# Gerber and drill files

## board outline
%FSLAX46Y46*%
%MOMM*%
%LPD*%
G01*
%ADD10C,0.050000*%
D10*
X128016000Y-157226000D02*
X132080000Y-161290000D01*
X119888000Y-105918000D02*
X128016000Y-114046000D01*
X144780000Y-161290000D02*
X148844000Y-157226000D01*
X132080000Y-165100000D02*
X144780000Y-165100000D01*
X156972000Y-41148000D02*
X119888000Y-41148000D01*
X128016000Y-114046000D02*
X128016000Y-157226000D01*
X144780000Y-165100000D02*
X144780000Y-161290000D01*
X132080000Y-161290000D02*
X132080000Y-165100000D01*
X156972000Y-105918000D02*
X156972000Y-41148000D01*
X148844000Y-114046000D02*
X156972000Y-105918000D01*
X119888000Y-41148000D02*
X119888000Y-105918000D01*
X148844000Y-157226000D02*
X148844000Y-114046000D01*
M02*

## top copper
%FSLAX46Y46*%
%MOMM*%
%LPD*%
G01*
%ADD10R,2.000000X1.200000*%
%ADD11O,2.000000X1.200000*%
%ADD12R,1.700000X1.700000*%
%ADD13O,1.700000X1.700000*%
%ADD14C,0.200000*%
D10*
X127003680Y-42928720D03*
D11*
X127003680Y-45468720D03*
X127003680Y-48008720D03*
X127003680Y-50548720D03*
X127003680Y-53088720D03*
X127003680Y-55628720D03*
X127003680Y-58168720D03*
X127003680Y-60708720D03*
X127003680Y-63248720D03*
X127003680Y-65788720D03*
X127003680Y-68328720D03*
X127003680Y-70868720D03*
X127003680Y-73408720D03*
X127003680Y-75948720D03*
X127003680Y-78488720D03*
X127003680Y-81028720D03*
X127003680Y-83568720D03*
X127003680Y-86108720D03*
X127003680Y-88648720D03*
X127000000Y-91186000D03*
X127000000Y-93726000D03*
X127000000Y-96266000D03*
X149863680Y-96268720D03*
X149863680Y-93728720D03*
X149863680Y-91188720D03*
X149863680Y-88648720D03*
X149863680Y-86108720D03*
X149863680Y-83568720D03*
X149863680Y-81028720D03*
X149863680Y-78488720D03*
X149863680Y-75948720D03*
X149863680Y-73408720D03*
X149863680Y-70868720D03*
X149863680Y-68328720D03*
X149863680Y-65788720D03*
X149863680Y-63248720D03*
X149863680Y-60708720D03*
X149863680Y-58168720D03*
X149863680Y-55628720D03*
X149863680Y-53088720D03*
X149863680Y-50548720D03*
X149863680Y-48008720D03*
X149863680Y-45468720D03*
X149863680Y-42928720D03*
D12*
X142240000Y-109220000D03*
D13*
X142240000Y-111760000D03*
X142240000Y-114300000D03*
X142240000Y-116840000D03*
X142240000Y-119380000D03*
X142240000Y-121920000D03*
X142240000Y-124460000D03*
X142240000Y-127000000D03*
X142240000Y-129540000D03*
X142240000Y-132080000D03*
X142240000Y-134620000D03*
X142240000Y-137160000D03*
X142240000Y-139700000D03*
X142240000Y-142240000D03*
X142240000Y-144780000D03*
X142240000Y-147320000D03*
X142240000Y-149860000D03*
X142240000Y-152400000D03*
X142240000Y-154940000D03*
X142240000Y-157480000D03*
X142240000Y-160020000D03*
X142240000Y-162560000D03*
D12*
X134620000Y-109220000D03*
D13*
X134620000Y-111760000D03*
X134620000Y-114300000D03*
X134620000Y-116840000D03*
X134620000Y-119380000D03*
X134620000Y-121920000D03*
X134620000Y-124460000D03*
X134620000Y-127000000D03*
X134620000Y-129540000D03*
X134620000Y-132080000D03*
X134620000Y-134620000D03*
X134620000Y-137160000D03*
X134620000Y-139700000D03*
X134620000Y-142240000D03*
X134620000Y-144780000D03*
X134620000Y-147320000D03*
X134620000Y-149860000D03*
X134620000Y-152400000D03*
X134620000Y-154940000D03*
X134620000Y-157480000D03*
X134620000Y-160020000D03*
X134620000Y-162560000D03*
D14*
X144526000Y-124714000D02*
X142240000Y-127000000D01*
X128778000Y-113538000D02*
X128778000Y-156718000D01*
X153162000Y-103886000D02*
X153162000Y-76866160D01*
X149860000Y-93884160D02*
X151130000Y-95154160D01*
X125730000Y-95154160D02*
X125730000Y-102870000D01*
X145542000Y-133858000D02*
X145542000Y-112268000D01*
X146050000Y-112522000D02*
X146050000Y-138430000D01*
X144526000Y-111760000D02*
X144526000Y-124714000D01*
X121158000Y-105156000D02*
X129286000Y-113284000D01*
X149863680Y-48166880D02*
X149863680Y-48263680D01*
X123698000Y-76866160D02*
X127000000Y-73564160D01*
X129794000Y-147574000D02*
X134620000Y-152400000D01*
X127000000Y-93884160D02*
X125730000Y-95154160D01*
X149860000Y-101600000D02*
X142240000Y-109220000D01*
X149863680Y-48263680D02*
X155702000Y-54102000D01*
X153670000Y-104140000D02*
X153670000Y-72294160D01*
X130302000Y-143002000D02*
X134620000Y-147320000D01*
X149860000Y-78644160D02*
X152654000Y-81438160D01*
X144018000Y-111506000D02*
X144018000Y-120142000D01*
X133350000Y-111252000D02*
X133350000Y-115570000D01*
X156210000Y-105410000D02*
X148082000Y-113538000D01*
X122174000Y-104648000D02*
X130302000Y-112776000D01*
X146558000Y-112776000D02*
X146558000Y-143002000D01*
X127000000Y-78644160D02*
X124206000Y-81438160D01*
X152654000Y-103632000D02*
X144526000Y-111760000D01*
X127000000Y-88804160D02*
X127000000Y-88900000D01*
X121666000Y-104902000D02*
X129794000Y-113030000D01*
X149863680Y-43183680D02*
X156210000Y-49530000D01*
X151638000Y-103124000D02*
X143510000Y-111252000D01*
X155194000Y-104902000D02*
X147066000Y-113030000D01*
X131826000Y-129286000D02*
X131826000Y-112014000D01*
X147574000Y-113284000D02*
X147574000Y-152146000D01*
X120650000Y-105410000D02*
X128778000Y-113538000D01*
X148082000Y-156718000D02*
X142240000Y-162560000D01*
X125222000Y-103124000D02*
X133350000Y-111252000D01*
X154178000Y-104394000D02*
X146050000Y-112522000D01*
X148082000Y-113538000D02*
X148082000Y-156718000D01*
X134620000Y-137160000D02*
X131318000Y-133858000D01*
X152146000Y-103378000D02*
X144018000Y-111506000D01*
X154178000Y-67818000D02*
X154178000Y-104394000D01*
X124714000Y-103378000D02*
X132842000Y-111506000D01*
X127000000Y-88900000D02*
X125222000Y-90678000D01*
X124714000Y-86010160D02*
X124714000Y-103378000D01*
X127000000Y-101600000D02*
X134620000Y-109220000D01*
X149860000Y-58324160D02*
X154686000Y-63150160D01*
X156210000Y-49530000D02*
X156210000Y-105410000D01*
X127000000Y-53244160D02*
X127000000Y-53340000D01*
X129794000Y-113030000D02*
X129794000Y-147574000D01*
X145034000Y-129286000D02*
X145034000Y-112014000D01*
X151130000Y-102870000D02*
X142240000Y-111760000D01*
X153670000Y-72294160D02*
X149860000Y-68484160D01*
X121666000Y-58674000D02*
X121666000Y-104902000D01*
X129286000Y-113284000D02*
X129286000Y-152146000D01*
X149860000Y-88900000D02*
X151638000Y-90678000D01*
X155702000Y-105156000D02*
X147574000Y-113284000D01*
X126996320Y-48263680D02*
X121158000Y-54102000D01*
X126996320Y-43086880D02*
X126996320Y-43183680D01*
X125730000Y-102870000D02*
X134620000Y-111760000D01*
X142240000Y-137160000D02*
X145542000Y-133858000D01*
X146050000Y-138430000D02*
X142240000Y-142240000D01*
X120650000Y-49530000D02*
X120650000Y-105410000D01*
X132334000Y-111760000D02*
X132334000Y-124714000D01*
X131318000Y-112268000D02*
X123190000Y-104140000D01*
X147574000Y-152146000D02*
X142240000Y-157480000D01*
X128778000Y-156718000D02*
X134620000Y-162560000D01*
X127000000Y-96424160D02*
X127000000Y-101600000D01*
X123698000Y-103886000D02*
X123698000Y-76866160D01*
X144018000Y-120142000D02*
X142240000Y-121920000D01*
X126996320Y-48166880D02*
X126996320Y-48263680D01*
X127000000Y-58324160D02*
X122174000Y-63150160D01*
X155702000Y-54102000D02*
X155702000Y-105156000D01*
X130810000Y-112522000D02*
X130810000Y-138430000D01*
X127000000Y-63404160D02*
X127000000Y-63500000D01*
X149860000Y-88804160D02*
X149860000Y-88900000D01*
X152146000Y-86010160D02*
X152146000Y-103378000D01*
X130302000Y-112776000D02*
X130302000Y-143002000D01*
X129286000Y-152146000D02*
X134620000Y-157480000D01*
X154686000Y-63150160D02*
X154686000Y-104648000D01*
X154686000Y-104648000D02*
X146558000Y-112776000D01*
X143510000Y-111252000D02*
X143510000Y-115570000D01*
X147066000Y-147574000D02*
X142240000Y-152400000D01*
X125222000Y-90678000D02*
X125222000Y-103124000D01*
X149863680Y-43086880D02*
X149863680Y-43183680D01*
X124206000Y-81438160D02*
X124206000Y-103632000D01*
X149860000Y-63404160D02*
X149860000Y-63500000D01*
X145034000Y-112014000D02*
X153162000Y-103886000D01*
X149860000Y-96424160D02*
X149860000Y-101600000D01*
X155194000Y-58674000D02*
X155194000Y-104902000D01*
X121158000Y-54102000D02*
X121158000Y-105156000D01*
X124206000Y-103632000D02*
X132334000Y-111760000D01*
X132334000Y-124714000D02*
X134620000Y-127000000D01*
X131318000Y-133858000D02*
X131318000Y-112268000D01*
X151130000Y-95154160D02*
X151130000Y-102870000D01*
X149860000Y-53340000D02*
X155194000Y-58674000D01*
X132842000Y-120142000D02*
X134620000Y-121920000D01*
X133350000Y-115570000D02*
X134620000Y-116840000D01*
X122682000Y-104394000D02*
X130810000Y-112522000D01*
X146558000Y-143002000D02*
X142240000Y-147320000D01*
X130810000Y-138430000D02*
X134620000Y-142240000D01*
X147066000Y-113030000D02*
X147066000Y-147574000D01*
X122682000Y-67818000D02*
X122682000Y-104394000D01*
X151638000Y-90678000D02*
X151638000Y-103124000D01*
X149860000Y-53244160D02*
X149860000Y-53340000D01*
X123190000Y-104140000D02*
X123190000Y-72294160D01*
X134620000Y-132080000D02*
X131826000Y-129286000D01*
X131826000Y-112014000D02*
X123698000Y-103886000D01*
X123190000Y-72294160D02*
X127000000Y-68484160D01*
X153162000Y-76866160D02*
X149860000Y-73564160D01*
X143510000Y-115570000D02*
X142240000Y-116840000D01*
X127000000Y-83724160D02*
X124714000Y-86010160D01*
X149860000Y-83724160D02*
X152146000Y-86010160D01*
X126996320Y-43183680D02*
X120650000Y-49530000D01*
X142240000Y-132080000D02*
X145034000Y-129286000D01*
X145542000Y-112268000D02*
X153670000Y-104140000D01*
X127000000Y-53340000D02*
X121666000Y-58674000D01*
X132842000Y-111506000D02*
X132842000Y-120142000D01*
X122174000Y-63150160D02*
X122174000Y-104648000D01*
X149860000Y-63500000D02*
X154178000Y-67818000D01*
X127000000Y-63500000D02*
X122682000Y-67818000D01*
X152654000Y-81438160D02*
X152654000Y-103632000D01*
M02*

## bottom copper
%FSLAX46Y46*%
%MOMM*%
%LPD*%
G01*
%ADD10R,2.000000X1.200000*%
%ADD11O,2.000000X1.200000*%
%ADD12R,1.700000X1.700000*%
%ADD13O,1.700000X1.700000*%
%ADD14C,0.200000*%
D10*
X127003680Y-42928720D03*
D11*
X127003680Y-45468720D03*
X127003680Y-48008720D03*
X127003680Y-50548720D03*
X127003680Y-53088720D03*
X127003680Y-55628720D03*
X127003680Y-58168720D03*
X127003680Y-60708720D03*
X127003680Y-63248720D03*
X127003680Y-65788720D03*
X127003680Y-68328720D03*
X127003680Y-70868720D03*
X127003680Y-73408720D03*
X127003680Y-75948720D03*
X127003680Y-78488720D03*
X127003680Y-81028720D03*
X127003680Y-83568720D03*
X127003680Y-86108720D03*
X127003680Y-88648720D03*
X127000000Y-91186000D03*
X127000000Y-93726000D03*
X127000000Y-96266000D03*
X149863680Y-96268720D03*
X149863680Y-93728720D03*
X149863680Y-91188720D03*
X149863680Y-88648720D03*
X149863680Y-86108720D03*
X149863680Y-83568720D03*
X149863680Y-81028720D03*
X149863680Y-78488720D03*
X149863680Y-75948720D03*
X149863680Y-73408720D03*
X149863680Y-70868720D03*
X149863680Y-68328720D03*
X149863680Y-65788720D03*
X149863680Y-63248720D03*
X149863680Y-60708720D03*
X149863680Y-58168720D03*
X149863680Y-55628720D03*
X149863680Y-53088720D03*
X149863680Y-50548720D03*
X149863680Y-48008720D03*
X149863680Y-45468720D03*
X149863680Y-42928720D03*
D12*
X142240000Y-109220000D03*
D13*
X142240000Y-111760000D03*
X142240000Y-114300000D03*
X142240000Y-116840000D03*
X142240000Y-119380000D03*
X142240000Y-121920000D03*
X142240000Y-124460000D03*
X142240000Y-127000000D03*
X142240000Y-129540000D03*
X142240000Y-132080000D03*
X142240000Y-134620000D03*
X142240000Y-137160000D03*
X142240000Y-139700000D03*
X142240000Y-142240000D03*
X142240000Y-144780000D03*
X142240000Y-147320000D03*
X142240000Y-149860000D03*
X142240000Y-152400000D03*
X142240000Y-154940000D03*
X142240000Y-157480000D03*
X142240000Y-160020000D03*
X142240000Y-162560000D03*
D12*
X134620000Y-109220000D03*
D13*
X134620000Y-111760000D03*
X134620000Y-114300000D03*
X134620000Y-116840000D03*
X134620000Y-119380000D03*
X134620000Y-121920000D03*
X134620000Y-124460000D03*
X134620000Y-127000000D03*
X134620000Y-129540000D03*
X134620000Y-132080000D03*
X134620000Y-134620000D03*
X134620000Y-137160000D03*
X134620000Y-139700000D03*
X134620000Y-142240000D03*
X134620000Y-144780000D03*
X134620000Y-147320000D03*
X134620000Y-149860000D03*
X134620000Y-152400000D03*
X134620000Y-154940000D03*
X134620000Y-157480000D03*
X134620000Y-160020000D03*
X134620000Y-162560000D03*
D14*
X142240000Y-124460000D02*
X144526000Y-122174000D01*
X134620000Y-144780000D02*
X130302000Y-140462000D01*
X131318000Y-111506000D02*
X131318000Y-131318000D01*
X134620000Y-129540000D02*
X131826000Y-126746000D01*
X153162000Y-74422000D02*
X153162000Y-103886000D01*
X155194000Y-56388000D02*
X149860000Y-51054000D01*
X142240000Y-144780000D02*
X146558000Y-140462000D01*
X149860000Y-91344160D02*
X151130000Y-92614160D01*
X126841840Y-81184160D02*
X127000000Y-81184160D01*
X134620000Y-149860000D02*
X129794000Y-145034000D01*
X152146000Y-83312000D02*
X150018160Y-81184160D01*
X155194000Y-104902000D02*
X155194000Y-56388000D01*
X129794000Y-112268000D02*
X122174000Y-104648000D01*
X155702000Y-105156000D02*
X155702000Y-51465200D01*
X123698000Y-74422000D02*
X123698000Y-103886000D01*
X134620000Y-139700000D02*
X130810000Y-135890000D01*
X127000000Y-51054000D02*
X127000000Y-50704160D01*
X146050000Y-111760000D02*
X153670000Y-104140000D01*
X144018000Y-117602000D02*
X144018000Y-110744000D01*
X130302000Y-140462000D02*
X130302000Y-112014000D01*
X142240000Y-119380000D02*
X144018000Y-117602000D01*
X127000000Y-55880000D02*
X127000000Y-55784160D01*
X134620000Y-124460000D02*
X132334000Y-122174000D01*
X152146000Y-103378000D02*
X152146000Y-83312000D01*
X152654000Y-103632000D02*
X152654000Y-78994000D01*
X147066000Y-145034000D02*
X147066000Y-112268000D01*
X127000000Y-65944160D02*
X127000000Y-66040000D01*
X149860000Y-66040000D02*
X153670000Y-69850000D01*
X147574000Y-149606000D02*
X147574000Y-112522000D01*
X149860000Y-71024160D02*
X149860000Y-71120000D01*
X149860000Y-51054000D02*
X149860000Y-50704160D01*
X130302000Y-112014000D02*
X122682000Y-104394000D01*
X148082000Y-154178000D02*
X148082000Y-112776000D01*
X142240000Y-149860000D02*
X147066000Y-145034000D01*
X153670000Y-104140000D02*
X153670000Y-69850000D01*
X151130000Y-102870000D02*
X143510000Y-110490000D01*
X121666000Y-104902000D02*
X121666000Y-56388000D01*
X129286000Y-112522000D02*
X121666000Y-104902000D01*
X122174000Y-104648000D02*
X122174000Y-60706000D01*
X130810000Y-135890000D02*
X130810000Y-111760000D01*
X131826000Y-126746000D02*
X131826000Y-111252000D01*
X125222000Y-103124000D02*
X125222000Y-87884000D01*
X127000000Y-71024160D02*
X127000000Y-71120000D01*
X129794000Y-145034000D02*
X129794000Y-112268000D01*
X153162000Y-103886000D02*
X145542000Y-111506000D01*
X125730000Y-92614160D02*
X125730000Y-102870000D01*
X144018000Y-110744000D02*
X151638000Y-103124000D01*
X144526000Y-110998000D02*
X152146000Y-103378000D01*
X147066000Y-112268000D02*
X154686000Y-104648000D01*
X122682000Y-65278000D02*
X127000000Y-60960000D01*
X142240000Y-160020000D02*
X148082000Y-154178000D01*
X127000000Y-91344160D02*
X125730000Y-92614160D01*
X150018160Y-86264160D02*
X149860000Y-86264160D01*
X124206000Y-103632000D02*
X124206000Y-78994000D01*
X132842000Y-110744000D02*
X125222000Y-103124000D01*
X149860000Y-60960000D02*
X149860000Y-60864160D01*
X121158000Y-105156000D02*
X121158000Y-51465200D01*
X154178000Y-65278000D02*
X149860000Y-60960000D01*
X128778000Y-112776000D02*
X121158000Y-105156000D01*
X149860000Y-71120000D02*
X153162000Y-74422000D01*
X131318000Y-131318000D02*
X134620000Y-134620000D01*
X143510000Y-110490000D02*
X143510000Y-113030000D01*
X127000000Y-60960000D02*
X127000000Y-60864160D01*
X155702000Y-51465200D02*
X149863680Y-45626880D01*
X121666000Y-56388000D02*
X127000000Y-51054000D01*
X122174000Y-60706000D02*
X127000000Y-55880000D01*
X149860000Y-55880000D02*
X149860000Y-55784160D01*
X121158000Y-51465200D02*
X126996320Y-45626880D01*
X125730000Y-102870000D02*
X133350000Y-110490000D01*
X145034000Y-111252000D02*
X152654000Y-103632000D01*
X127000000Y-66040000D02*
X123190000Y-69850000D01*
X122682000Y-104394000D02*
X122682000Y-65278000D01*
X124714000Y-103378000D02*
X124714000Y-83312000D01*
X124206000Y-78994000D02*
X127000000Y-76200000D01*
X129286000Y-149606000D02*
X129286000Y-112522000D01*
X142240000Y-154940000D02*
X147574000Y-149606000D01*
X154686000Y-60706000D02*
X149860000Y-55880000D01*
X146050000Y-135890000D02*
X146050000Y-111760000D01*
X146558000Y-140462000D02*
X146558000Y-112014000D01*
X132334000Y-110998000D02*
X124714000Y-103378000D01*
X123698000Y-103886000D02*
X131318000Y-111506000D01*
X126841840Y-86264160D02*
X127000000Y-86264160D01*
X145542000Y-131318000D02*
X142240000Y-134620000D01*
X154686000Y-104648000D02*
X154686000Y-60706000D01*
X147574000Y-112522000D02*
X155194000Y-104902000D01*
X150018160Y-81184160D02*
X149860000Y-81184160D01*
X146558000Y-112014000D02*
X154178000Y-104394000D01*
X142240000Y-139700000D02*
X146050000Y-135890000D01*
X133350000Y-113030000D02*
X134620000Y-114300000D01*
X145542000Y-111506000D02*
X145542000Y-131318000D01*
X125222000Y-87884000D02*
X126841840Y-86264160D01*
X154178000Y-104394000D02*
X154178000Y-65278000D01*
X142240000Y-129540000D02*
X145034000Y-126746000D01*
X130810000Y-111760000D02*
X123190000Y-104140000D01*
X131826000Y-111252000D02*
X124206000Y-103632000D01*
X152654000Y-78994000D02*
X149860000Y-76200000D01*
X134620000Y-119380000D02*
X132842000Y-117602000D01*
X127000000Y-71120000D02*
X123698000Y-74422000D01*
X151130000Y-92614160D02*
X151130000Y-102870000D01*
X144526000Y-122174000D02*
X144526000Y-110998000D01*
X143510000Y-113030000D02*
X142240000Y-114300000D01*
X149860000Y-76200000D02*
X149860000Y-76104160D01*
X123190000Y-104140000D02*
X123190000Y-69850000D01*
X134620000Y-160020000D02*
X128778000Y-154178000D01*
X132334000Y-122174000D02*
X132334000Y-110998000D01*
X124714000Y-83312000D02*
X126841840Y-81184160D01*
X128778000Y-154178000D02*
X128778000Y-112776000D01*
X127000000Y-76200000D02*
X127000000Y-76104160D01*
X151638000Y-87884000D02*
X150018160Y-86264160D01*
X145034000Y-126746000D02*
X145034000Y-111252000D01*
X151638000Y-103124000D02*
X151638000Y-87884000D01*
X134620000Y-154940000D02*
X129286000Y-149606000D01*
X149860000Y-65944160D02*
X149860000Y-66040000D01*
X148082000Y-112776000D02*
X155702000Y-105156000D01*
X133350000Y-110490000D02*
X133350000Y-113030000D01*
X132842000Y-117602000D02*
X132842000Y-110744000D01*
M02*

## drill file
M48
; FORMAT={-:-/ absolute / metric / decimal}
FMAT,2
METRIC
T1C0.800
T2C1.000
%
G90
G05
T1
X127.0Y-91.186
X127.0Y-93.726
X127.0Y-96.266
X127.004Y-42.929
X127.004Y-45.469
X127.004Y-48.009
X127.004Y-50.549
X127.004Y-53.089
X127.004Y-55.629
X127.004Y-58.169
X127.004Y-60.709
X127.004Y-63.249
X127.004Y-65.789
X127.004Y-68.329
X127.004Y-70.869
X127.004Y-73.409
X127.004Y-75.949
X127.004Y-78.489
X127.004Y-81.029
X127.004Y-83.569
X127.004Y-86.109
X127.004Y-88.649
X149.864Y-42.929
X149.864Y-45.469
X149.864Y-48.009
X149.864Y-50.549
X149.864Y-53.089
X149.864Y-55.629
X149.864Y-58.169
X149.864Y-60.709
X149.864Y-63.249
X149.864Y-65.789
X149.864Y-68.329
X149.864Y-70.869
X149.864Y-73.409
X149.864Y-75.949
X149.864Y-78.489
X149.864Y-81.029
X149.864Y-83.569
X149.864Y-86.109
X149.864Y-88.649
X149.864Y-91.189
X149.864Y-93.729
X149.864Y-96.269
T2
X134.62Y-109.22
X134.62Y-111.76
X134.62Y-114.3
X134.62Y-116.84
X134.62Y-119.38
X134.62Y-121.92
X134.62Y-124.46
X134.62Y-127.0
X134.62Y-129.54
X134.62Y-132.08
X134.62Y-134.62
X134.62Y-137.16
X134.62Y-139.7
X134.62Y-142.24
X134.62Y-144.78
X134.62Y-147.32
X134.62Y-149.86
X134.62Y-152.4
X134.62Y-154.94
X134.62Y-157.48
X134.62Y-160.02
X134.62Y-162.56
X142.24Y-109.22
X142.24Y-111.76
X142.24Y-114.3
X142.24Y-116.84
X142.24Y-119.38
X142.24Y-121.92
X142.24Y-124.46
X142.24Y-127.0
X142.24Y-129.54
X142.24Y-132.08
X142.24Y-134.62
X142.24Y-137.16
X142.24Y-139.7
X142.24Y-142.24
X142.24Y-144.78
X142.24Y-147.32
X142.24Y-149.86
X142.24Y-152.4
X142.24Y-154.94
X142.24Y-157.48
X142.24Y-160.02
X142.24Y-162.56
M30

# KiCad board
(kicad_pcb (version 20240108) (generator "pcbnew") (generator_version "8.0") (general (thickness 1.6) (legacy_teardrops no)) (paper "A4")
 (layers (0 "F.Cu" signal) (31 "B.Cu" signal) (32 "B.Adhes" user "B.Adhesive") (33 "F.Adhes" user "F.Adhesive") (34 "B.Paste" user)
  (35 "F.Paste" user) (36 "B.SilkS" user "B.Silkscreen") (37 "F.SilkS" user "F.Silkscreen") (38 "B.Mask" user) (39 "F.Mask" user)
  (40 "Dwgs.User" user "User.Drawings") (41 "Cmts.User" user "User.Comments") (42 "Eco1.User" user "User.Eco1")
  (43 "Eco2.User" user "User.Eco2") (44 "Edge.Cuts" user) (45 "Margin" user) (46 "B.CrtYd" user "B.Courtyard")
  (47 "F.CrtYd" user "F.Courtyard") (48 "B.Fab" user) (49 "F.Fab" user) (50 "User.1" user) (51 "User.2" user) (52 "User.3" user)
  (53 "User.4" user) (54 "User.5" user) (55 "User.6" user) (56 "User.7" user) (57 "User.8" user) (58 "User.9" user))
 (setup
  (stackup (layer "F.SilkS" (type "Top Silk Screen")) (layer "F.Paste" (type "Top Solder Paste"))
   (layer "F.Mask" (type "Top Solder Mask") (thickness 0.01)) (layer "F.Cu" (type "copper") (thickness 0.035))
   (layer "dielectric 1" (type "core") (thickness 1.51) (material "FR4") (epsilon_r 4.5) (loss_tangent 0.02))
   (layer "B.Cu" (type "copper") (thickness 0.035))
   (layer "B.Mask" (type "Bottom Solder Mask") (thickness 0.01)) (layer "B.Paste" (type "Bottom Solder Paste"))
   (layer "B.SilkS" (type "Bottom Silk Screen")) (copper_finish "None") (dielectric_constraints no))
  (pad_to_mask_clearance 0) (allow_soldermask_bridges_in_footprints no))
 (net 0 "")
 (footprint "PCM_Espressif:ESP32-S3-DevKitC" (layer "F.Cu") (at 127.00368 42.92872)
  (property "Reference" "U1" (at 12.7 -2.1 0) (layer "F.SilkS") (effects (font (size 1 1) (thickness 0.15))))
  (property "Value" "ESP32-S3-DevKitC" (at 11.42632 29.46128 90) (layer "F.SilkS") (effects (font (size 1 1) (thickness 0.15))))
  (pad "1" thru_hole rect (at 0 0 270) (size 1.2 2) (drill 0.8) (layers "*.Cu" "*.Mask") (remove_unused_layers no))
  (pad "2" thru_hole oval (at 0 2.54 270) (size 1.2 2) (drill 0.8) (layers "*.Cu" "*.Mask") (remove_unused_layers no))
  (pad "3" thru_hole oval (at 0 5.08 270) (size 1.2 2) (drill 0.8) (layers "*.Cu" "*.Mask") (remove_unused_layers no))
  (pad "4" thru_hole oval (at 0 7.62 270) (size 1.2 2) (drill 0.8) (layers "*.Cu" "*.Mask") (remove_unused_layers no))
  (pad "5" thru_hole oval (at 0 10.16 270) (size 1.2 2) (drill 0.8) (layers "*.Cu" "*.Mask") (remove_unused_layers no))
  (pad "6" thru_hole oval (at 0 12.7 270) (size 1.2 2) (drill 0.8) (layers "*.Cu" "*.Mask") (remove_unused_layers no))
  (pad "7" thru_hole oval (at 0 15.24 270) (size 1.2 2) (drill 0.8) (layers "*.Cu" "*.Mask") (remove_unused_layers no))
  (pad "8" thru_hole oval (at 0 17.78 270) (size 1.2 2) (drill 0.8) (layers "*.Cu" "*.Mask") (remove_unused_layers no))
  (pad "9" thru_hole oval (at 0 20.32 270) (size 1.2 2) (drill 0.8) (layers "*.Cu" "*.Mask") (remove_unused_layers no))
  (pad "10" thru_hole oval (at 0 22.86 270) (size 1.2 2) (drill 0.8) (layers "*.Cu" "*.Mask") (remove_unused_layers no))
  (pad "11" thru_hole oval (at 0 25.4 270) (size 1.2 2) (drill 0.8) (layers "*.Cu" "*.Mask") (remove_unused_layers no))
  (pad "12" thru_hole oval (at 0 27.94 270) (size 1.2 2) (drill 0.8) (layers "*.Cu" "*.Mask") (remove_unused_layers no))
  (pad "13" thru_hole oval (at 0 30.48 270) (size 1.2 2) (drill 0.8) (layers "*.Cu" "*.Mask") (remove_unused_layers no))
  (pad "14" thru_hole oval (at 0 33.02 270) (size 1.2 2) (drill 0.8) (layers "*.Cu" "*.Mask") (remove_unused_layers no))
  (pad "15" thru_hole oval (at 0 35.56 270) (size 1.2 2) (drill 0.8) (layers "*.Cu" "*.Mask") (remove_unused_layers no))
  (pad "16" thru_hole oval (at 0 38.1 270) (size 1.2 2) (drill 0.8) (layers "*.Cu" "*.Mask") (remove_unused_layers no))
  (pad "17" thru_hole oval (at 0 40.64 270) (size 1.2 2) (drill 0.8) (layers "*.Cu" "*.Mask") (remove_unused_layers no))
  (pad "18" thru_hole oval (at 0 43.18 270) (size 1.2 2) (drill 0.8) (layers "*.Cu" "*.Mask") (remove_unused_layers no))
  (pad "19" thru_hole oval (at 0 45.72 270) (size 1.2 2) (drill 0.8) (layers "*.Cu" "*.Mask") (remove_unused_layers no))
  (pad "20" thru_hole oval (at -0.00368 48.25728 270) (size 1.2 2) (drill 0.8) (layers "*.Cu" "*.Mask") (remove_unused_layers no))
  (pad "21" thru_hole oval (at -0.00368 50.79728 270) (size 1.2 2) (drill 0.8) (layers "*.Cu" "*.Mask") (remove_unused_layers no))
  (pad "22" thru_hole oval (at -0.00368 53.33728 270) (size 1.2 2) (drill 0.8) (layers "*.Cu" "*.Mask") (remove_unused_layers no))
  (pad "23" thru_hole oval (at 22.86 53.34 270) (size 1.2 2) (drill 0.8) (layers "*.Cu" "*.Mask") (remove_unused_layers no))
  (pad "24" thru_hole oval (at 22.86 50.8 270) (size 1.2 2) (drill 0.8) (layers "*.Cu" "*.Mask") (remove_unused_layers no))
  (pad "25" thru_hole oval (at 22.86 48.26 270) (size 1.2 2) (drill 0.8) (layers "*.Cu" "*.Mask") (remove_unused_layers no))
  (pad "26" thru_hole oval (at 22.86 45.72 270) (size 1.2 2) (drill 0.8) (layers "*.Cu" "*.Mask") (remove_unused_layers no))
  (pad "27" thru_hole oval (at 22.86 43.18 270) (size 1.2 2) (drill 0.8) (layers "*.Cu" "*.Mask") (remove_unused_layers no))
  (pad "28" thru_hole oval (at 22.86 40.64 270) (size 1.2 2) (drill 0.8) (layers "*.Cu" "*.Mask") (remove_unused_layers no))
  (pad "29" thru_hole oval (at 22.86 38.1 270) (size 1.2 2) (drill 0.8) (layers "*.Cu" "*.Mask") (remove_unused_layers no))
  (pad "30" thru_hole oval (at 22.86 35.56 270) (size 1.2 2) (drill 0.8) (layers "*.Cu" "*.Mask") (remove_unused_layers no))
  (pad "31" thru_hole oval (at 22.86 33.02 270) (size 1.2 2) (drill 0.8) (layers "*.Cu" "*.Mask") (remove_unused_layers no))
  (pad "32" thru_hole oval (at 22.86 30.48 270) (size 1.2 2) (drill 0.8) (layers "*.Cu" "*.Mask") (remove_unused_layers no))
  (pad "33" thru_hole oval (at 22.86 27.94 270) (size 1.2 2) (drill 0.8) (layers "*.Cu" "*.Mask") (remove_unused_layers no))
  (pad "34" thru_hole oval (at 22.86 25.4 270) (size 1.2 2) (drill 0.8) (layers "*.Cu" "*.Mask") (remove_unused_layers no))
  (pad "35" thru_hole oval (at 22.86 22.86 270) (size 1.2 2) (drill 0.8) (layers "*.Cu" "*.Mask") (remove_unused_layers no))
  (pad "36" thru_hole oval (at 22.86 20.32 270) (size 1.2 2) (drill 0.8) (layers "*.Cu" "*.Mask") (remove_unused_layers no))
  (pad "37" thru_hole oval (at 22.86 17.78 270) (size 1.2 2) (drill 0.8) (layers "*.Cu" "*.Mask") (remove_unused_layers no))
  (pad "38" thru_hole oval (at 22.86 15.24 270) (size 1.2 2) (drill 0.8) (layers "*.Cu" "*.Mask") (remove_unused_layers no))
  (pad "39" thru_hole oval (at 22.86 12.7 270) (size 1.2 2) (drill 0.8) (layers "*.Cu" "*.Mask") (remove_unused_layers no))
  (pad "40" thru_hole oval (at 22.86 10.16 270) (size 1.2 2) (drill 0.8) (layers "*.Cu" "*.Mask") (remove_unused_layers no))
  (pad "41" thru_hole oval (at 22.86 7.62 270) (size 1.2 2) (drill 0.8) (layers "*.Cu" "*.Mask") (remove_unused_layers no))
  (pad "42" thru_hole oval (at 22.86 5.08 270) (size 1.2 2) (drill 0.8) (layers "*.Cu" "*.Mask") (remove_unused_layers no))
  (pad "43" thru_hole oval (at 22.86 2.54 270) (size 1.2 2) (drill 0.8) (layers "*.Cu" "*.Mask") (remove_unused_layers no))
  (pad "44" thru_hole oval (at 22.86 0 270) (size 1.2 2) (drill 0.8) (layers "*.Cu" "*.Mask") (remove_unused_layers no)))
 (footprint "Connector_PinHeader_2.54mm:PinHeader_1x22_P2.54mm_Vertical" (layer "B.Cu") (at 142.24 109.22 180)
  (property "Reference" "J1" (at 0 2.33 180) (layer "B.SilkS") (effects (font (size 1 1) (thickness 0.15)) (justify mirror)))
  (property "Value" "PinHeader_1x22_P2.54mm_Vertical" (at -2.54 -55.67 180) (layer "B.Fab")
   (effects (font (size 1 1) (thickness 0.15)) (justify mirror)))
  (pad "1" thru_hole rect (at 0 0 180) (size 1.7 1.7) (drill 1) (layers "*.Cu" "*.Mask") (remove_unused_layers no))
  (pad "2" thru_hole oval (at 0 -2.54 180) (size 1.7 1.7) (drill 1) (layers "*.Cu" "*.Mask") (remove_unused_layers no))
  (pad "3" thru_hole oval (at 0 -5.08 180) (size 1.7 1.7) (drill 1) (layers "*.Cu" "*.Mask") (remove_unused_layers no))
  (pad "4" thru_hole oval (at 0 -7.62 180) (size 1.7 1.7) (drill 1) (layers "*.Cu" "*.Mask") (remove_unused_layers no))
  (pad "5" thru_hole oval (at 0 -10.16 180) (size 1.7 1.7) (drill 1) (layers "*.Cu" "*.Mask") (remove_unused_layers no))
  (pad "6" thru_hole oval (at 0 -12.7 180) (size 1.7 1.7) (drill 1) (layers "*.Cu" "*.Mask") (remove_unused_layers no))
  (pad "7" thru_hole oval (at 0 -15.24 180) (size 1.7 1.7) (drill 1) (layers "*.Cu" "*.Mask") (remove_unused_layers no))
  (pad "8" thru_hole oval (at 0 -17.78 180) (size 1.7 1.7) (drill 1) (layers "*.Cu" "*.Mask") (remove_unused_layers no))
  (pad "9" thru_hole oval (at 0 -20.32 180) (size 1.7 1.7) (drill 1) (layers "*.Cu" "*.Mask") (remove_unused_layers no))
  (pad "10" thru_hole oval (at 0 -22.86 180) (size 1.7 1.7) (drill 1) (layers "*.Cu" "*.Mask") (remove_unused_layers no))
  (pad "11" thru_hole oval (at 0 -25.4 180) (size 1.7 1.7) (drill 1) (layers "*.Cu" "*.Mask") (remove_unused_layers no))
  (pad "12" thru_hole oval (at 0 -27.94 180) (size 1.7 1.7) (drill 1) (layers "*.Cu" "*.Mask") (remove_unused_layers no))
  (pad "13" thru_hole oval (at 0 -30.48 180) (size 1.7 1.7) (drill 1) (layers "*.Cu" "*.Mask") (remove_unused_layers no))
  (pad "14" thru_hole oval (at 0 -33.02 180) (size 1.7 1.7) (drill 1) (layers "*.Cu" "*.Mask") (remove_unused_layers no))
  (pad "15" thru_hole oval (at 0 -35.56 180) (size 1.7 1.7) (drill 1) (layers "*.Cu" "*.Mask") (remove_unused_layers no))
  (pad "16" thru_hole oval (at 0 -38.1 180) (size 1.7 1.7) (drill 1) (layers "*.Cu" "*.Mask") (remove_unused_layers no))
  (pad "17" thru_hole oval (at 0 -40.64 180) (size 1.7 1.7) (drill 1) (layers "*.Cu" "*.Mask") (remove_unused_layers no))
  (pad "18" thru_hole oval (at 0 -43.18 180) (size 1.7 1.7) (drill 1) (layers "*.Cu" "*.Mask") (remove_unused_layers no))
  (pad "19" thru_hole oval (at 0 -45.72 180) (size 1.7 1.7) (drill 1) (layers "*.Cu" "*.Mask") (remove_unused_layers no))
  (pad "20" thru_hole oval (at 0 -48.26 180) (size 1.7 1.7) (drill 1) (layers "*.Cu" "*.Mask") (remove_unused_layers no))
  (pad "21" thru_hole oval (at 0 -50.8 180) (size 1.7 1.7) (drill 1) (layers "*.Cu" "*.Mask") (remove_unused_layers no))
  (pad "22" thru_hole oval (at 0 -53.34 180) (size 1.7 1.7) (drill 1) (layers "*.Cu" "*.Mask") (remove_unused_layers no)))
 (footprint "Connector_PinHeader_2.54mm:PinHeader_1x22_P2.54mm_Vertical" (layer "B.Cu") (at 134.62 109.22 180)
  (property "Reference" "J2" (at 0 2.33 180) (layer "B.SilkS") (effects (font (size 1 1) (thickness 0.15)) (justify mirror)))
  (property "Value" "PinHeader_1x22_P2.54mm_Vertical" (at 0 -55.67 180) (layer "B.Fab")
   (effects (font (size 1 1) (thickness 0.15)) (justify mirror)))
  (pad "1" thru_hole rect (at 0 0 180) (size 1.7 1.7) (drill 1) (layers "*.Cu" "*.Mask") (remove_unused_layers no))
  (pad "2" thru_hole oval (at 0 -2.54 180) (size 1.7 1.7) (drill 1) (layers "*.Cu" "*.Mask") (remove_unused_layers no))
  (pad "3" thru_hole oval (at 0 -5.08 180) (size 1.7 1.7) (drill 1) (layers "*.Cu" "*.Mask") (remove_unused_layers no))
  (pad "4" thru_hole oval (at 0 -7.62 180) (size 1.7 1.7) (drill 1) (layers "*.Cu" "*.Mask") (remove_unused_layers no))
  (pad "5" thru_hole oval (at 0 -10.16 180) (size 1.7 1.7) (drill 1) (layers "*.Cu" "*.Mask") (remove_unused_layers no))
  (pad "6" thru_hole oval (at 0 -12.7 180) (size 1.7 1.7) (drill 1) (layers "*.Cu" "*.Mask") (remove_unused_layers no))
  (pad "7" thru_hole oval (at 0 -15.24 180) (size 1.7 1.7) (drill 1) (layers "*.Cu" "*.Mask") (remove_unused_layers no))
  (pad "8" thru_hole oval (at 0 -17.78 180) (size 1.7 1.7) (drill 1) (layers "*.Cu" "*.Mask") (remove_unused_layers no))
  (pad "9" thru_hole oval (at 0 -20.32 180) (size 1.7 1.7) (drill 1) (layers "*.Cu" "*.Mask") (remove_unused_layers no))
  (pad "10" thru_hole oval (at 0 -22.86 180) (size 1.7 1.7) (drill 1) (layers "*.Cu" "*.Mask") (remove_unused_layers no))
  (pad "11" thru_hole oval (at 0 -25.4 180) (size 1.7 1.7) (drill 1) (layers "*.Cu" "*.Mask") (remove_unused_layers no))
  (pad "12" thru_hole oval (at 0 -27.94 180) (size 1.7 1.7) (drill 1) (layers "*.Cu" "*.Mask") (remove_unused_layers no))
  (pad "13" thru_hole oval (at 0 -30.48 180) (size 1.7 1.7) (drill 1) (layers "*.Cu" "*.Mask") (remove_unused_layers no))
  (pad "14" thru_hole oval (at 0 -33.02 180) (size 1.7 1.7) (drill 1) (layers "*.Cu" "*.Mask") (remove_unused_layers no))
  (pad "15" thru_hole oval (at 0 -35.56 180) (size 1.7 1.7) (drill 1) (layers "*.Cu" "*.Mask") (remove_unused_layers no))
  (pad "16" thru_hole oval (at 0 -38.1 180) (size 1.7 1.7) (drill 1) (layers "*.Cu" "*.Mask") (remove_unused_layers no))
  (pad "17" thru_hole oval (at 0 -40.64 180) (size 1.7 1.7) (drill 1) (layers "*.Cu" "*.Mask") (remove_unused_layers no))
  (pad "18" thru_hole oval (at 0 -43.18 180) (size 1.7 1.7) (drill 1) (layers "*.Cu" "*.Mask") (remove_unused_layers no))
  (pad "19" thru_hole oval (at 0 -45.72 180) (size 1.7 1.7) (drill 1) (layers "*.Cu" "*.Mask") (remove_unused_layers no))
  (pad "20" thru_hole oval (at 0 -48.26 180) (size 1.7 1.7) (drill 1) (layers "*.Cu" "*.Mask") (remove_unused_layers no))
  (pad "21" thru_hole oval (at 0 -50.8 180) (size 1.7 1.7) (drill 1) (layers "*.Cu" "*.Mask") (remove_unused_layers no))
  (pad "22" thru_hole oval (at 0 -53.34 180) (size 1.7 1.7) (drill 1) (layers "*.Cu" "*.Mask") (remove_unused_layers no)))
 (gr_line (start 128.016 157.226) (end 132.08 161.29) (stroke (width 0.05) (type default)) (layer "Edge.Cuts"))
 (gr_line (start 119.888 105.918) (end 128.016 114.046) (stroke (width 0.05) (type default)) (layer "Edge.Cuts"))
 (gr_line (start 144.78 161.29) (end 148.844 157.226) (stroke (width 0.05) (type default)) (layer "Edge.Cuts"))
 (gr_line (start 132.08 165.1) (end 144.78 165.1) (stroke (width 0.05) (type default)) (layer "Edge.Cuts"))
 (gr_line (start 156.972 41.148) (end 119.888 41.148) (stroke (width 0.05) (type default)) (layer "Edge.Cuts"))
 (gr_line (start 128.016 114.046) (end 128.016 157.226) (stroke (width 0.05) (type default)) (layer "Edge.Cuts"))
 (gr_line (start 144.78 165.1) (end 144.78 161.29) (stroke (width 0.05) (type default)) (layer "Edge.Cuts"))
 (gr_line (start 132.08 161.29) (end 132.08 165.1) (stroke (width 0.05) (type default)) (layer "Edge.Cuts"))
 (gr_line (start 156.972 105.918) (end 156.972 41.148) (stroke (width 0.05) (type default)) (layer "Edge.Cuts"))
 (gr_line (start 148.844 114.046) (end 156.972 105.918) (stroke (width 0.05) (type default)) (layer "Edge.Cuts"))
 (gr_line (start 119.888 41.148) (end 119.888 105.918) (stroke (width 0.05) (type default)) (layer "Edge.Cuts"))
 (gr_line (start 148.844 157.226) (end 148.844 114.046) (stroke (width 0.05) (type default)) (layer "Edge.Cuts"))
 (segment (start 144.526 124.714) (end 142.24 127) (width 0.2) (layer "F.Cu") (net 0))
 (segment (start 128.778 113.538) (end 128.778 156.718) (width 0.2) (layer "F.Cu") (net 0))
 (segment (start 153.162 103.886) (end 153.162 76.86616) (width 0.2) (layer "F.Cu") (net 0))
 (segment (start 149.86 93.88416) (end 151.13 95.15416) (width 0.2) (layer "F.Cu") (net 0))
 (segment (start 125.73 95.15416) (end 125.73 102.87) (width 0.2) (layer "F.Cu") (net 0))
 (segment (start 145.542 133.858) (end 145.542 112.268) (width 0.2) (layer "F.Cu") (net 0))
 (segment (start 146.05 112.522) (end 146.05 138.43) (width 0.2) (layer "F.Cu") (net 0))
 (segment (start 144.526 111.76) (end 144.526 124.714) (width 0.2) (layer "F.Cu") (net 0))
 (segment (start 121.158 105.156) (end 129.286 113.284) (width 0.2) (layer "F.Cu") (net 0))
 (segment (start 149.86368 48.16688) (end 149.86368 48.26368) (width 0.2) (layer "F.Cu") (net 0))
 (segment (start 123.698 76.86616) (end 127 73.56416) (width 0.2) (layer "F.Cu") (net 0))
 (segment (start 129.794 147.574) (end 134.62 152.4) (width 0.2) (layer "F.Cu") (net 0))
 (segment (start 127 93.88416) (end 125.73 95.15416) (width 0.2) (layer "F.Cu") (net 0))
 (segment (start 149.86 101.6) (end 142.24 109.22) (width 0.2) (layer "F.Cu") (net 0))
 (segment (start 149.86368 48.26368) (end 155.702 54.102) (width 0.2) (layer "F.Cu") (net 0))
 (segment (start 153.67 104.14) (end 153.67 72.29416) (width 0.2) (layer "F.Cu") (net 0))
 (segment (start 130.302 143.002) (end 134.62 147.32) (width 0.2) (layer "F.Cu") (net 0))
 (segment (start 149.86 78.64416) (end 152.654 81.43816) (width 0.2) (layer "F.Cu") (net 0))
 (segment (start 144.018 111.506) (end 144.018 120.142) (width 0.2) (layer "F.Cu") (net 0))
 (segment (start 133.35 111.252) (end 133.35 115.57) (width 0.2) (layer "F.Cu") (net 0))
 (segment (start 156.21 105.41) (end 148.082 113.538) (width 0.2) (layer "F.Cu") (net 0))
 (segment (start 122.174 104.648) (end 130.302 112.776) (width 0.2) (layer "F.Cu") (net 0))
 (segment (start 146.558 112.776) (end 146.558 143.002) (width 0.2) (layer "F.Cu") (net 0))
 (segment (start 127 78.64416) (end 124.206 81.43816) (width 0.2) (layer "F.Cu") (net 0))
 (segment (start 152.654 103.632) (end 144.526 111.76) (width 0.2) (layer "F.Cu") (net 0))
 (segment (start 127 88.80416) (end 127 88.9) (width 0.2) (layer "F.Cu") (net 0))
 (segment (start 121.666 104.902) (end 129.794 113.03) (width 0.2) (layer "F.Cu") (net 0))
 (segment (start 149.86368 43.18368) (end 156.21 49.53) (width 0.2) (layer "F.Cu") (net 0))
 (segment (start 151.638 103.124) (end 143.51 111.252) (width 0.2) (layer "F.Cu") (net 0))
 (segment (start 155.194 104.902) (end 147.066 113.03) (width 0.2) (layer "F.Cu") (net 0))
 (segment (start 131.826 129.286) (end 131.826 112.014) (width 0.2) (layer "F.Cu") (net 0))
 (segment (start 147.574 113.284) (end 147.574 152.146) (width 0.2) (layer "F.Cu") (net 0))
 (segment (start 120.65 105.41) (end 128.778 113.538) (width 0.2) (layer "F.Cu") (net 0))
 (segment (start 148.082 156.718) (end 142.24 162.56) (width 0.2) (layer "F.Cu") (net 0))
 (segment (start 125.222 103.124) (end 133.35 111.252) (width 0.2) (layer "F.Cu") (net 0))
 (segment (start 154.178 104.394) (end 146.05 112.522) (width 0.2) (layer "F.Cu") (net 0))
 (segment (start 148.082 113.538) (end 148.082 156.718) (width 0.2) (layer "F.Cu") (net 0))
 (segment (start 134.62 137.16) (end 131.318 133.858) (width 0.2) (layer "F.Cu") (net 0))
 (segment (start 152.146 103.378) (end 144.018 111.506) (width 0.2) (layer "F.Cu") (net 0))
 (segment (start 154.178 67.818) (end 154.178 104.394) (width 0.2) (layer "F.Cu") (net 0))
 (segment (start 124.714 103.378) (end 132.842 111.506) (width 0.2) (layer "F.Cu") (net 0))
 (segment (start 127 88.9) (end 125.222 90.678) (width 0.2) (layer "F.Cu") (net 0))
 (segment (start 124.714 86.01016) (end 124.714 103.378) (width 0.2) (layer "F.Cu") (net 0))
 (segment (start 127 101.6) (end 134.62 109.22) (width 0.2) (layer "F.Cu") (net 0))
 (segment (start 149.86 58.32416) (end 154.686 63.15016) (width 0.2) (layer "F.Cu") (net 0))
 (segment (start 156.21 49.53) (end 156.21 105.41) (width 0.2) (layer "F.Cu") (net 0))
 (segment (start 127 53.24416) (end 127 53.34) (width 0.2) (layer "F.Cu") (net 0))
 (segment (start 129.794 113.03) (end 129.794 147.574) (width 0.2) (layer "F.Cu") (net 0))
 (segment (start 145.034 129.286) (end 145.034 112.014) (width 0.2) (layer "F.Cu") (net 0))
 (segment (start 151.13 102.87) (end 142.24 111.76) (width 0.2) (layer "F.Cu") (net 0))
 (segment (start 153.67 72.29416) (end 149.86 68.48416) (width 0.2) (layer "F.Cu") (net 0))
 (segment (start 121.666 58.674) (end 121.666 104.902) (width 0.2) (layer "F.Cu") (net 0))
 (segment (start 129.286 113.284) (end 129.286 152.146) (width 0.2) (layer "F.Cu") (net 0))
 (segment (start 149.86 88.9) (end 151.638 90.678) (width 0.2) (layer "F.Cu") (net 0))
 (segment (start 155.702 105.156) (end 147.574 113.284) (width 0.2) (layer "F.Cu") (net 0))
 (segment (start 126.99632 48.26368) (end 121.158 54.102) (width 0.2) (layer "F.Cu") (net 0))
 (segment (start 126.99632 43.08688) (end 126.99632 43.18368) (width 0.2) (layer "F.Cu") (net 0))
 (segment (start 125.73 102.87) (end 134.62 111.76) (width 0.2) (layer "F.Cu") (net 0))
 (segment (start 142.24 137.16) (end 145.542 133.858) (width 0.2) (layer "F.Cu") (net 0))
 (segment (start 146.05 138.43) (end 142.24 142.24) (width 0.2) (layer "F.Cu") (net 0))
 (segment (start 120.65 49.53) (end 120.65 105.41) (width 0.2) (layer "F.Cu") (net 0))
 (segment (start 132.334 111.76) (end 132.334 124.714) (width 0.2) (layer "F.Cu") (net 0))
 (segment (start 131.318 112.268) (end 123.19 104.14) (width 0.2) (layer "F.Cu") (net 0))
 (segment (start 147.574 152.146) (end 142.24 157.48) (width 0.2) (layer "F.Cu") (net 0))
 (segment (start 128.778 156.718) (end 134.62 162.56) (width 0.2) (layer "F.Cu") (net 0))
 (segment (start 127 96.42416) (end 127 101.6) (width 0.2) (layer "F.Cu") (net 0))
 (segment (start 123.698 103.886) (end 123.698 76.86616) (width 0.2) (layer "F.Cu") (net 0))
 (segment (start 144.018 120.142) (end 142.24 121.92) (width 0.2) (layer "F.Cu") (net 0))
 (segment (start 126.99632 48.16688) (end 126.99632 48.26368) (width 0.2) (layer "F.Cu") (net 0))
 (segment (start 127 58.32416) (end 122.174 63.15016) (width 0.2) (layer "F.Cu") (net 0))
 (segment (start 155.702 54.102) (end 155.702 105.156) (width 0.2) (layer "F.Cu") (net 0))
 (segment (start 130.81 112.522) (end 130.81 138.43) (width 0.2) (layer "F.Cu") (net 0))
 (segment (start 127 63.40416) (end 127 63.5) (width 0.2) (layer "F.Cu") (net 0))
 (segment (start 149.86 88.80416) (end 149.86 88.9) (width 0.2) (layer "F.Cu") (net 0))
 (segment (start 152.146 86.01016) (end 152.146 103.378) (width 0.2) (layer "F.Cu") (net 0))
 (segment (start 130.302 112.776) (end 130.302 143.002) (width 0.2) (layer "F.Cu") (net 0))
 (segment (start 129.286 152.146) (end 134.62 157.48) (width 0.2) (layer "F.Cu") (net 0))
 (segment (start 154.686 63.15016) (end 154.686 104.648) (width 0.2) (layer "F.Cu") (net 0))
 (segment (start 154.686 104.648) (end 146.558 112.776) (width 0.2) (layer "F.Cu") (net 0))
 (segment (start 143.51 111.252) (end 143.51 115.57) (width 0.2) (layer "F.Cu") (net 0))
 (segment (start 147.066 147.574) (end 142.24 152.4) (width 0.2) (layer "F.Cu") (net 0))
 (segment (start 125.222 90.678) (end 125.222 103.124) (width 0.2) (layer "F.Cu") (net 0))
 (segment (start 149.86368 43.08688) (end 149.86368 43.18368) (width 0.2) (layer "F.Cu") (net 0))
 (segment (start 124.206 81.43816) (end 124.206 103.632) (width 0.2) (layer "F.Cu") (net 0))
 (segment (start 149.86 63.40416) (end 149.86 63.5) (width 0.2) (layer "F.Cu") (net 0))
 (segment (start 145.034 112.014) (end 153.162 103.886) (width 0.2) (layer "F.Cu") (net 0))
 (segment (start 149.86 96.42416) (end 149.86 101.6) (width 0.2) (layer "F.Cu") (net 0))
 (segment (start 155.194 58.674) (end 155.194 104.902) (width 0.2) (layer "F.Cu") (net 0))
 (segment (start 121.158 54.102) (end 121.158 105.156) (width 0.2) (layer "F.Cu") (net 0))
 (segment (start 124.206 103.632) (end 132.334 111.76) (width 0.2) (layer "F.Cu") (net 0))
 (segment (start 132.334 124.714) (end 134.62 127) (width 0.2) (layer "F.Cu") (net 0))
 (segment (start 131.318 133.858) (end 131.318 112.268) (width 0.2) (layer "F.Cu") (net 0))
 (segment (start 151.13 95.15416) (end 151.13 102.87) (width 0.2) (layer "F.Cu") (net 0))
 (segment (start 149.86 53.34) (end 155.194 58.674) (width 0.2) (layer "F.Cu") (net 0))
 (segment (start 132.842 120.142) (end 134.62 121.92) (width 0.2) (layer "F.Cu") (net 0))
 (segment (start 133.35 115.57) (end 134.62 116.84) (width 0.2) (layer "F.Cu") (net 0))
 (segment (start 122.682 104.394) (end 130.81 112.522) (width 0.2) (layer "F.Cu") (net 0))
 (segment (start 146.558 143.002) (end 142.24 147.32) (width 0.2) (layer "F.Cu") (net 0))
 (segment (start 130.81 138.43) (end 134.62 142.24) (width 0.2) (layer "F.Cu") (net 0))
 (segment (start 147.066 113.03) (end 147.066 147.574) (width 0.2) (layer "F.Cu") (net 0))
 (segment (start 122.682 67.818) (end 122.682 104.394) (width 0.2) (layer "F.Cu") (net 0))
 (segment (start 151.638 90.678) (end 151.638 103.124) (width 0.2) (layer "F.Cu") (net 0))
 (segment (start 149.86 53.24416) (end 149.86 53.34) (width 0.2) (layer "F.Cu") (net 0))
 (segment (start 123.19 104.14) (end 123.19 72.29416) (width 0.2) (layer "F.Cu") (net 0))
 (segment (start 134.62 132.08) (end 131.826 129.286) (width 0.2) (layer "F.Cu") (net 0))
 (segment (start 131.826 112.014) (end 123.698 103.886) (width 0.2) (layer "F.Cu") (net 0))
 (segment (start 123.19 72.29416) (end 127 68.48416) (width 0.2) (layer "F.Cu") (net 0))
 (segment (start 153.162 76.86616) (end 149.86 73.56416) (width 0.2) (layer "F.Cu") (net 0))
 (segment (start 143.51 115.57) (end 142.24 116.84) (width 0.2) (layer "F.Cu") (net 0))
 (segment (start 127 83.72416) (end 124.714 86.01016) (width 0.2) (layer "F.Cu") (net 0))
 (segment (start 149.86 83.72416) (end 152.146 86.01016) (width 0.2) (layer "F.Cu") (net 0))
 (segment (start 126.99632 43.18368) (end 120.65 49.53) (width 0.2) (layer "F.Cu") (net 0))
 (segment (start 142.24 132.08) (end 145.034 129.286) (width 0.2) (layer "F.Cu") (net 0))
 (segment (start 145.542 112.268) (end 153.67 104.14) (width 0.2) (layer "F.Cu") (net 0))
 (segment (start 127 53.34) (end 121.666 58.674) (width 0.2) (layer "F.Cu") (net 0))
 (segment (start 132.842 111.506) (end 132.842 120.142) (width 0.2) (layer "F.Cu") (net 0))
 (segment (start 122.174 63.15016) (end 122.174 104.648) (width 0.2) (layer "F.Cu") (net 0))
 (segment (start 149.86 63.5) (end 154.178 67.818) (width 0.2) (layer "F.Cu") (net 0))
 (segment (start 127 63.5) (end 122.682 67.818) (width 0.2) (layer "F.Cu") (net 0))
 (segment (start 152.654 81.43816) (end 152.654 103.632) (width 0.2) (layer "F.Cu") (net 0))
 (segment (start 142.24 124.46) (end 144.526 122.174) (width 0.2) (layer "B.Cu") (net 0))
 (segment (start 134.62 144.78) (end 130.302 140.462) (width 0.2) (layer "B.Cu") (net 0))
 (segment (start 131.318 111.506) (end 131.318 131.318) (width 0.2) (layer "B.Cu") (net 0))
 (segment (start 134.62 129.54) (end 131.826 126.746) (width 0.2) (layer "B.Cu") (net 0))
 (segment (start 153.162 74.422) (end 153.162 103.886) (width 0.2) (layer "B.Cu") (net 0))
 (segment (start 155.194 56.388) (end 149.86 51.054) (width 0.2) (layer "B.Cu") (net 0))
 (segment (start 142.24 144.78) (end 146.558 140.462) (width 0.2) (layer "B.Cu") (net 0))
 (segment (start 149.86 91.34416) (end 151.13 92.61416) (width 0.2) (layer "B.Cu") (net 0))
 (segment (start 126.84184 81.18416) (end 127 81.18416) (width 0.2) (layer "B.Cu") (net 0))
 (segment (start 134.62 149.86) (end 129.794 145.034) (width 0.2) (layer "B.Cu") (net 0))
 (segment (start 152.146 83.312) (end 150.01816 81.18416) (width 0.2) (layer "B.Cu") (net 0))
 (segment (start 155.194 104.902) (end 155.194 56.388) (width 0.2) (layer "B.Cu") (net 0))
 (segment (start 129.794 112.268) (end 122.174 104.648) (width 0.2) (layer "B.Cu") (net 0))
 (segment (start 155.702 105.156) (end 155.702 51.4652) (width 0.2) (layer "B.Cu") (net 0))
 (segment (start 123.698 74.422) (end 123.698 103.886) (width 0.2) (layer "B.Cu") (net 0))
 (segment (start 134.62 139.7) (end 130.81 135.89) (width 0.2) (layer "B.Cu") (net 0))
 (segment (start 127 51.054) (end 127 50.70416) (width 0.2) (layer "B.Cu") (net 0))
 (segment (start 146.05 111.76) (end 153.67 104.14) (width 0.2) (layer "B.Cu") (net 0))
 (segment (start 144.018 117.602) (end 144.018 110.744) (width 0.2) (layer "B.Cu") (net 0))
 (segment (start 130.302 140.462) (end 130.302 112.014) (width 0.2) (layer "B.Cu") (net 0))
 (segment (start 142.24 119.38) (end 144.018 117.602) (width 0.2) (layer "B.Cu") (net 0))
 (segment (start 127 55.88) (end 127 55.78416) (width 0.2) (layer "B.Cu") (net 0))
 (segment (start 134.62 124.46) (end 132.334 122.174) (width 0.2) (layer "B.Cu") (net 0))
 (segment (start 152.146 103.378) (end 152.146 83.312) (width 0.2) (layer "B.Cu") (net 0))
 (segment (start 152.654 103.632) (end 152.654 78.994) (width 0.2) (layer "B.Cu") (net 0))
 (segment (start 147.066 145.034) (end 147.066 112.268) (width 0.2) (layer "B.Cu") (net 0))
 (segment (start 127 65.94416) (end 127 66.04) (width 0.2) (layer "B.Cu") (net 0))
 (segment (start 149.86 66.04) (end 153.67 69.85) (width 0.2) (layer "B.Cu") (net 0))
 (segment (start 147.574 149.606) (end 147.574 112.522) (width 0.2) (layer "B.Cu") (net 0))
 (segment (start 149.86 71.02416) (end 149.86 71.12) (width 0.2) (layer "B.Cu") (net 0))
 (segment (start 149.86 51.054) (end 149.86 50.70416) (width 0.2) (layer "B.Cu") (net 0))
 (segment (start 130.302 112.014) (end 122.682 104.394) (width 0.2) (layer "B.Cu") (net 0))
 (segment (start 148.082 154.178) (end 148.082 112.776) (width 0.2) (layer "B.Cu") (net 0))
 (segment (start 142.24 149.86) (end 147.066 145.034) (width 0.2) (layer "B.Cu") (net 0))
 (segment (start 153.67 104.14) (end 153.67 69.85) (width 0.2) (layer "B.Cu") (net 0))
 (segment (start 151.13 102.87) (end 143.51 110.49) (width 0.2) (layer "B.Cu") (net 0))
 (segment (start 121.666 104.902) (end 121.666 56.388) (width 0.2) (layer "B.Cu") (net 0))
 (segment (start 129.286 112.522) (end 121.666 104.902) (width 0.2) (layer "B.Cu") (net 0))
 (segment (start 122.174 104.648) (end 122.174 60.706) (width 0.2) (layer "B.Cu") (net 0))
 (segment (start 130.81 135.89) (end 130.81 111.76) (width 0.2) (layer "B.Cu") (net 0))
 (segment (start 131.826 126.746) (end 131.826 111.252) (width 0.2) (layer "B.Cu") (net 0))
 (segment (start 125.222 103.124) (end 125.222 87.884) (width 0.2) (layer "B.Cu") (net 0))
 (segment (start 127 71.02416) (end 127 71.12) (width 0.2) (layer "B.Cu") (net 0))
 (segment (start 129.794 145.034) (end 129.794 112.268) (width 0.2) (layer "B.Cu") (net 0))
 (segment (start 153.162 103.886) (end 145.542 111.506) (width 0.2) (layer "B.Cu") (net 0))
 (segment (start 125.73 92.61416) (end 125.73 102.87) (width 0.2) (layer "B.Cu") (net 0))
 (segment (start 144.018 110.744) (end 151.638 103.124) (width 0.2) (layer "B.Cu") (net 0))
 (segment (start 144.526 110.998) (end 152.146 103.378) (width 0.2) (layer "B.Cu") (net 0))
 (segment (start 147.066 112.268) (end 154.686 104.648) (width 0.2) (layer "B.Cu") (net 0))
 (segment (start 122.682 65.278) (end 127 60.96) (width 0.2) (layer "B.Cu") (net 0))
 (segment (start 142.24 160.02) (end 148.082 154.178) (width 0.2) (layer "B.Cu") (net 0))
 (segment (start 127 91.34416) (end 125.73 92.61416) (width 0.2) (layer "B.Cu") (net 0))
 (segment (start 150.01816 86.26416) (end 149.86 86.26416) (width 0.2) (layer "B.Cu") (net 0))
 (segment (start 124.206 103.632) (end 124.206 78.994) (width 0.2) (layer "B.Cu") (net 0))
 (segment (start 132.842 110.744) (end 125.222 103.124) (width 0.2) (layer "B.Cu") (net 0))
 (segment (start 149.86 60.96) (end 149.86 60.86416) (width 0.2) (layer "B.Cu") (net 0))
 (segment (start 121.158 105.156) (end 121.158 51.4652) (width 0.2) (layer "B.Cu") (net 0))
 (segment (start 154.178 65.278) (end 149.86 60.96) (width 0.2) (layer "B.Cu") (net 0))
 (segment (start 128.778 112.776) (end 121.158 105.156) (width 0.2) (layer "B.Cu") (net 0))
 (segment (start 149.86 71.12) (end 153.162 74.422) (width 0.2) (layer "B.Cu") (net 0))
 (segment (start 131.318 131.318) (end 134.62 134.62) (width 0.2) (layer "B.Cu") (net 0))
 (segment (start 143.51 110.49) (end 143.51 113.03) (width 0.2) (layer "B.Cu") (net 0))
 (segment (start 127 60.96) (end 127 60.86416) (width 0.2) (layer "B.Cu") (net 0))
 (segment (start 155.702 51.4652) (end 149.86368 45.62688) (width 0.2) (layer "B.Cu") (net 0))
 (segment (start 121.666 56.388) (end 127 51.054) (width 0.2) (layer "B.Cu") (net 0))
 (segment (start 122.174 60.706) (end 127 55.88) (width 0.2) (layer "B.Cu") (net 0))
 (segment (start 149.86 55.88) (end 149.86 55.78416) (width 0.2) (layer "B.Cu") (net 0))
 (segment (start 121.158 51.4652) (end 126.99632 45.62688) (width 0.2) (layer "B.Cu") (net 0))
 (segment (start 125.73 102.87) (end 133.35 110.49) (width 0.2) (layer "B.Cu") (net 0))
 (segment (start 145.034 111.252) (end 152.654 103.632) (width 0.2) (layer "B.Cu") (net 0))
 (segment (start 127 66.04) (end 123.19 69.85) (width 0.2) (layer "B.Cu") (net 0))
 (segment (start 122.682 104.394) (end 122.682 65.278) (width 0.2) (layer "B.Cu") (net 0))
 (segment (start 124.714 103.378) (end 124.714 83.312) (width 0.2) (layer "B.Cu") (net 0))
 (segment (start 124.206 78.994) (end 127 76.2) (width 0.2) (layer "B.Cu") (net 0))
 (segment (start 129.286 149.606) (end 129.286 112.522) (width 0.2) (layer "B.Cu") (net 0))
 (segment (start 142.24 154.94) (end 147.574 149.606) (width 0.2) (layer "B.Cu") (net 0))
 (segment (start 154.686 60.706) (end 149.86 55.88) (width 0.2) (layer "B.Cu") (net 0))
 (segment (start 146.05 135.89) (end 146.05 111.76) (width 0.2) (layer "B.Cu") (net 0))
 (segment (start 146.558 140.462) (end 146.558 112.014) (width 0.2) (layer "B.Cu") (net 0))
 (segment (start 132.334 110.998) (end 124.714 103.378) (width 0.2) (layer "B.Cu") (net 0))
 (segment (start 123.698 103.886) (end 131.318 111.506) (width 0.2) (layer "B.Cu") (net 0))
 (segment (start 126.84184 86.26416) (end 127 86.26416) (width 0.2) (layer "B.Cu") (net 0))
 (segment (start 145.542 131.318) (end 142.24 134.62) (width 0.2) (layer "B.Cu") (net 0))
 (segment (start 154.686 104.648) (end 154.686 60.706) (width 0.2) (layer "B.Cu") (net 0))
 (segment (start 147.574 112.522) (end 155.194 104.902) (width 0.2) (layer "B.Cu") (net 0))
 (segment (start 150.01816 81.18416) (end 149.86 81.18416) (width 0.2) (layer "B.Cu") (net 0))
 (segment (start 146.558 112.014) (end 154.178 104.394) (width 0.2) (layer "B.Cu") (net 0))
 (segment (start 142.24 139.7) (end 146.05 135.89) (width 0.2) (layer "B.Cu") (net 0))
 (segment (start 133.35 113.03) (end 134.62 114.3) (width 0.2) (layer "B.Cu") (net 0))
 (segment (start 145.542 111.506) (end 145.542 131.318) (width 0.2) (layer "B.Cu") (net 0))
 (segment (start 125.222 87.884) (end 126.84184 86.26416) (width 0.2) (layer "B.Cu") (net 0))
 (segment (start 154.178 104.394) (end 154.178 65.278) (width 0.2) (layer "B.Cu") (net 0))
 (segment (start 142.24 129.54) (end 145.034 126.746) (width 0.2) (layer "B.Cu") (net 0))
 (segment (start 130.81 111.76) (end 123.19 104.14) (width 0.2) (layer "B.Cu") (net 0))
 (segment (start 131.826 111.252) (end 124.206 103.632) (width 0.2) (layer "B.Cu") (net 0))
 (segment (start 152.654 78.994) (end 149.86 76.2) (width 0.2) (layer "B.Cu") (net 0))
 (segment (start 134.62 119.38) (end 132.842 117.602) (width 0.2) (layer "B.Cu") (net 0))
 (segment (start 127 71.12) (end 123.698 74.422) (width 0.2) (layer "B.Cu") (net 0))
 (segment (start 151.13 92.61416) (end 151.13 102.87) (width 0.2) (layer "B.Cu") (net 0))
 (segment (start 144.526 122.174) (end 144.526 110.998) (width 0.2) (layer "B.Cu") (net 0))
 (segment (start 143.51 113.03) (end 142.24 114.3) (width 0.2) (layer "B.Cu") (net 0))
 (segment (start 149.86 76.2) (end 149.86 76.10416) (width 0.2) (layer "B.Cu") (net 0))
 (segment (start 123.19 104.14) (end 123.19 69.85) (width 0.2) (layer "B.Cu") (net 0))
 (segment (start 134.62 160.02) (end 128.778 154.178) (width 0.2) (layer "B.Cu") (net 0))
 (segment (start 132.334 122.174) (end 132.334 110.998) (width 0.2) (layer "B.Cu") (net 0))
 (segment (start 124.714 83.312) (end 126.84184 81.18416) (width 0.2) (layer "B.Cu") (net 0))
 (segment (start 128.778 154.178) (end 128.778 112.776) (width 0.2) (layer "B.Cu") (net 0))
 (segment (start 127 76.2) (end 127 76.10416) (width 0.2) (layer "B.Cu") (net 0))
 (segment (start 151.638 87.884) (end 150.01816 86.26416) (width 0.2) (layer "B.Cu") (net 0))
 (segment (start 145.034 126.746) (end 145.034 111.252) (width 0.2) (layer "B.Cu") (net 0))
 (segment (start 151.638 103.124) (end 151.638 87.884) (width 0.2) (layer "B.Cu") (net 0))
 (segment (start 134.62 154.94) (end 129.286 149.606) (width 0.2) (layer "B.Cu") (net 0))
 (segment (start 149.86 65.94416) (end 149.86 66.04) (width 0.2) (layer "B.Cu") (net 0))
 (segment (start 148.082 112.776) (end 155.702 105.156) (width 0.2) (layer "B.Cu") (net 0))
 (segment (start 133.35 110.49) (end 133.35 113.03) (width 0.2) (layer "B.Cu") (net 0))
 (segment (start 132.842 117.602) (end 132.842 110.744) (width 0.2) (layer "B.Cu") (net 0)))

